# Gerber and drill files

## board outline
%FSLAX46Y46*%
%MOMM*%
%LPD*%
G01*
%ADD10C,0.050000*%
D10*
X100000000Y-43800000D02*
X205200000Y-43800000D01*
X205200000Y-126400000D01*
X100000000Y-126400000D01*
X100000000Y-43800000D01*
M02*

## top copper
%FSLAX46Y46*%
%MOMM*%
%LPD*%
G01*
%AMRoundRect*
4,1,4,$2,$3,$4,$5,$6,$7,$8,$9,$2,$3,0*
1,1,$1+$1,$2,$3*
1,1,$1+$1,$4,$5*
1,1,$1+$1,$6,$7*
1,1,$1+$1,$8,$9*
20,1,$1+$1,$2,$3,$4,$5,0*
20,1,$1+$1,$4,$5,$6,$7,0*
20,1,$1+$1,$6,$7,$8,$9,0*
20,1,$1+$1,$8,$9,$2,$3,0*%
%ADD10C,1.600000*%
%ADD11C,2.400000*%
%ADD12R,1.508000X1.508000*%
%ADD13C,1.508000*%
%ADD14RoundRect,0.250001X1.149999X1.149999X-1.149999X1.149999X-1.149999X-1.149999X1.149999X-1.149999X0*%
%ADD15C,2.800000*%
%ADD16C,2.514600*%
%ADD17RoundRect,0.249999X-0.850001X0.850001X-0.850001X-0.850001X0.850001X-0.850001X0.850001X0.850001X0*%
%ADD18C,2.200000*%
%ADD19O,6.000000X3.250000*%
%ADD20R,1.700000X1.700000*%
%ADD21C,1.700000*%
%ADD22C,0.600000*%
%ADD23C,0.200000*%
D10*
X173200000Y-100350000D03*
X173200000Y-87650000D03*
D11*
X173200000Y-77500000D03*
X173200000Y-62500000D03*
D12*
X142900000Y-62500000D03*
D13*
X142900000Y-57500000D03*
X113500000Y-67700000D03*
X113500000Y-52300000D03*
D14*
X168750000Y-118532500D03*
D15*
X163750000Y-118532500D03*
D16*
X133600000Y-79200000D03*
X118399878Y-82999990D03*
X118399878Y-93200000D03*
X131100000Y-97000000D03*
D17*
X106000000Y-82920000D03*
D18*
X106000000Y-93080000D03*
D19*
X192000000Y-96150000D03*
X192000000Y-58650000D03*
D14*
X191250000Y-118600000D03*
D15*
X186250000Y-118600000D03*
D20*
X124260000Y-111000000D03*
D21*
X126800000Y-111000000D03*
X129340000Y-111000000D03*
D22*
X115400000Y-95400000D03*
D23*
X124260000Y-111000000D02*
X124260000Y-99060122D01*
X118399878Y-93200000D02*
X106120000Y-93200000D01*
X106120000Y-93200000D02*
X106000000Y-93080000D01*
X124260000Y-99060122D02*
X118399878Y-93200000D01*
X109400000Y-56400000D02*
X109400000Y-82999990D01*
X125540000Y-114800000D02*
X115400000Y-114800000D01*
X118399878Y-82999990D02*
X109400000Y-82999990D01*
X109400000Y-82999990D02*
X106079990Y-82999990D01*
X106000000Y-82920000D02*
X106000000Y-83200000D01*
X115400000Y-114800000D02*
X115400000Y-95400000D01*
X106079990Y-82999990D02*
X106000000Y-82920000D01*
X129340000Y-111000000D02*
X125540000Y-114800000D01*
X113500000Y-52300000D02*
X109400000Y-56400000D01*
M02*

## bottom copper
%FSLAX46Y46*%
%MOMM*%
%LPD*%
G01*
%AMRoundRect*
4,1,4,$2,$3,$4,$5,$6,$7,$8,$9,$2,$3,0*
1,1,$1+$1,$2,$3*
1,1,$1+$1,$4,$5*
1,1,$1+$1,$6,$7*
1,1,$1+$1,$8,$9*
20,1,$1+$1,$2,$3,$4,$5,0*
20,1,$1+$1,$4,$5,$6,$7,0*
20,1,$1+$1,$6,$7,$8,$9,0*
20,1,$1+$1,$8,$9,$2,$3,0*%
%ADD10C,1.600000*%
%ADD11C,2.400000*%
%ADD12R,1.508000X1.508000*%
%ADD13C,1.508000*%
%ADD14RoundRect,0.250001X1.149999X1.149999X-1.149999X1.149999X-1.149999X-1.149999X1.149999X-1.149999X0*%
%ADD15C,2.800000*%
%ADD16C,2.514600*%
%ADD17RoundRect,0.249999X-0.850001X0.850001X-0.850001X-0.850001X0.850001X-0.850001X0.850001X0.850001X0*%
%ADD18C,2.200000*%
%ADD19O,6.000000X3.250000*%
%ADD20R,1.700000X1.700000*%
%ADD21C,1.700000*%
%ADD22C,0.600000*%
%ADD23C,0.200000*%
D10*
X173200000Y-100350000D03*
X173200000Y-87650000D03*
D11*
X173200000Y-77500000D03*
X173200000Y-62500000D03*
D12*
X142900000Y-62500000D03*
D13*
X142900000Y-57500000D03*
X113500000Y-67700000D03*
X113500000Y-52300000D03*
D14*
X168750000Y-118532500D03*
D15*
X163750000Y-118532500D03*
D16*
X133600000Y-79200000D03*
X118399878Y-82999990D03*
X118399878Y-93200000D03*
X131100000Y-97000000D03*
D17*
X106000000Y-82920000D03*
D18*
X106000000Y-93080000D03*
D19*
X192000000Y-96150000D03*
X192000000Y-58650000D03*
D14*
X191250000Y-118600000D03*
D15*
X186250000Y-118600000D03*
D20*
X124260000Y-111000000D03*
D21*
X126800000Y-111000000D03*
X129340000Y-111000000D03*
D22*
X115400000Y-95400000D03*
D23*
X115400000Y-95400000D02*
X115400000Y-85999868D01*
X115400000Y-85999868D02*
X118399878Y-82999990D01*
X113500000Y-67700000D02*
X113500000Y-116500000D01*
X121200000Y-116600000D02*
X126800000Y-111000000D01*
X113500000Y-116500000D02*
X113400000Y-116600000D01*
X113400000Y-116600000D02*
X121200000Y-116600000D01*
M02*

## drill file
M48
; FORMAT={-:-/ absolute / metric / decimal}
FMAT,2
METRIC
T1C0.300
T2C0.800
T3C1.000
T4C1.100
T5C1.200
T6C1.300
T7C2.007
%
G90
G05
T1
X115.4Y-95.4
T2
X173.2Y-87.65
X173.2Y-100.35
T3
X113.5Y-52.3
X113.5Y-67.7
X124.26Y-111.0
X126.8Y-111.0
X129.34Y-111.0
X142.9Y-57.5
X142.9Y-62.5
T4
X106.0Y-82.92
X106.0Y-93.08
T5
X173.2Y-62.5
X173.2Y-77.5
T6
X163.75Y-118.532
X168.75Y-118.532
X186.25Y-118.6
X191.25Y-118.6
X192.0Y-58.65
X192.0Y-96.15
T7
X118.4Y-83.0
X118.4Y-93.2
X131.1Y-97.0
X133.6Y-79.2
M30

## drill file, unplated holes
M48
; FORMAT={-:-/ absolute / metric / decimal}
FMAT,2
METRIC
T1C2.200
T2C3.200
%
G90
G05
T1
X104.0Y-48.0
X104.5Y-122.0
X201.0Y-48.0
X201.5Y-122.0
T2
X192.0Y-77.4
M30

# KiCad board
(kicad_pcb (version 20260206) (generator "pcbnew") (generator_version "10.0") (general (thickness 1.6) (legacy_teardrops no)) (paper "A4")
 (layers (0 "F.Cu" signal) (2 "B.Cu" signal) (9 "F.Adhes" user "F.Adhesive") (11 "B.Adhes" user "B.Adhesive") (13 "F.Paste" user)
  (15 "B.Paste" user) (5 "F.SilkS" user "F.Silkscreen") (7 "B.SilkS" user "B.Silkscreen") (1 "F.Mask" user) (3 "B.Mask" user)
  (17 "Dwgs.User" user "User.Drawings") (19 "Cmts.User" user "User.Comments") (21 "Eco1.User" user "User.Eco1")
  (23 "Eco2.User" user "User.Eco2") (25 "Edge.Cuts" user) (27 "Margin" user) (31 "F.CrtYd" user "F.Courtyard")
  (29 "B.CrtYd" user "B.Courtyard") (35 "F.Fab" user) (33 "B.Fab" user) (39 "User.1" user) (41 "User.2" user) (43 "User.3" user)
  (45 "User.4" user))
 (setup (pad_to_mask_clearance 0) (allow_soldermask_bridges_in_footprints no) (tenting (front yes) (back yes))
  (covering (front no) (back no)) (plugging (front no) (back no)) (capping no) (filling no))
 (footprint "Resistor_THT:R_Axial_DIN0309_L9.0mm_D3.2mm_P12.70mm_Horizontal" (layer "F.Cu") (at 173.2 100.35 90)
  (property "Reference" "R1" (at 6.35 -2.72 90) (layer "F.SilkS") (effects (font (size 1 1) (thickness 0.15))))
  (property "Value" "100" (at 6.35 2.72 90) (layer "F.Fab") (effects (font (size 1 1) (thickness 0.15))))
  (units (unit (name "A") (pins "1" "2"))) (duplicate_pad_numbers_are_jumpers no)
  (pad "1" thru_hole circle (at 0 0 90) (size 1.6 1.6) (drill 0.8) (layers "*.Cu" "*.Mask") (remove_unused_layers no) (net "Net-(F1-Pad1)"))
  (pad "2" thru_hole circle (at 12.7 0 90) (size 1.6 1.6) (drill 0.8) (layers "*.Cu" "*.Mask") (remove_unused_layers no)
   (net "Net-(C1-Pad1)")))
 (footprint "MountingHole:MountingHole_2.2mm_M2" (layer "F.Cu") (at 104.5 122)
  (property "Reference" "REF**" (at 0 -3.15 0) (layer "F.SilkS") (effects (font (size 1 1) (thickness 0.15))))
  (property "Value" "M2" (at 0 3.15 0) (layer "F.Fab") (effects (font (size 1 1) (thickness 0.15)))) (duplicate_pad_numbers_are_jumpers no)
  (pad "" np_thru_hole circle (at 0 0) (size 2.2 2.2) (drill 2.2) (layers "*.Cu" "*.Mask")))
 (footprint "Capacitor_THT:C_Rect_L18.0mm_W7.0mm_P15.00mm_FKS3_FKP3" (layer "F.Cu") (at 173.2 77.5 90)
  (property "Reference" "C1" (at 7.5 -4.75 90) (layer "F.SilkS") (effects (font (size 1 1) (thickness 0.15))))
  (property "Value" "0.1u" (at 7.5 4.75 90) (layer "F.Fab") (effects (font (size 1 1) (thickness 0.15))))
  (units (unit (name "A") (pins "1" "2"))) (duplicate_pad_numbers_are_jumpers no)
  (pad "1" thru_hole circle (at 0 0 90) (size 2.4 2.4) (drill 1.2) (layers "*.Cu" "*.Mask") (remove_unused_layers no) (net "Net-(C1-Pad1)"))
  (pad "2" thru_hole circle (at 15 0 90) (size 2.4 2.4) (drill 1.2) (layers "*.Cu" "*.Mask") (remove_unused_layers no)
   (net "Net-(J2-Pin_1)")))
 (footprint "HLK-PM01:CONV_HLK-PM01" (layer "F.Cu") (at 128.2 60 180)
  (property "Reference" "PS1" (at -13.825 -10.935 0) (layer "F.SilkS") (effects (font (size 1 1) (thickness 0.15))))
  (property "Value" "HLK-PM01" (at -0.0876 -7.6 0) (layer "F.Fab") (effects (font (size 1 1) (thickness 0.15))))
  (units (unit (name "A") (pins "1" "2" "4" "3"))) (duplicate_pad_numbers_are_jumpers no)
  (pad "1" thru_hole rect (at -14.7 -2.5 180) (size 1.508 1.508) (drill 1) (layers "*.Cu" "*.Mask") (remove_unused_layers no)
   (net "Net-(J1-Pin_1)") (solder_mask_margin 0.102))
  (pad "2" thru_hole circle (at -14.7 2.5 180) (size 1.508 1.508) (drill 1) (layers "*.Cu" "*.Mask") (remove_unused_layers no)
   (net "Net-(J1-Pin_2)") (solder_mask_margin 0.102))
  (pad "3" thru_hole circle (at 14.7 -7.7 180) (size 1.508 1.508) (drill 1) (layers "*.Cu" "*.Mask") (remove_unused_layers no)
   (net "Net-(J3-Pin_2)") (solder_mask_margin 0.102))
  (pad "4" thru_hole circle (at 14.7 7.7 180) (size 1.508 1.508) (drill 1) (layers "*.Cu" "*.Mask") (remove_unused_layers no)
   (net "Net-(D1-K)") (solder_mask_margin 0.102)))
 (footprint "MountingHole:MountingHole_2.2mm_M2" (layer "F.Cu") (at 104 48)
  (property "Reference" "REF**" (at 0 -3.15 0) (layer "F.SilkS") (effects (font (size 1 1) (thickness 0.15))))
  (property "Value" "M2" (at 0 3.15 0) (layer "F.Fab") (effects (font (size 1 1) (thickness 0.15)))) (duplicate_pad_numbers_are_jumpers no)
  (pad "" np_thru_hole circle (at 0 0) (size 2.2 2.2) (drill 2.2) (layers "*.Cu" "*.Mask")))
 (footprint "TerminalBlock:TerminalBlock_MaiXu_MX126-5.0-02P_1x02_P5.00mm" (layer "F.Cu") (at 168.75 118.5325 180)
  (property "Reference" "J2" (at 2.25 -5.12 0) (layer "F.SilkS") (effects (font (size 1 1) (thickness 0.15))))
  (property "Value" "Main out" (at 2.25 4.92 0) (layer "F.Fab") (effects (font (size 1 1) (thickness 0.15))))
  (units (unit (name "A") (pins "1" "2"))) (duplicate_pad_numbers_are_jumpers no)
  (pad "1" thru_hole roundrect (at 0 0 180) (size 2.8 2.8) (drill 1.3) (layers "*.Cu" "*.Mask") (remove_unused_layers no)
   (roundrect_rratio 0.089286) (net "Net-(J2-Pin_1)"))
  (pad "2" thru_hole circle (at 5 0 180) (size 2.8 2.8) (drill 1.3) (layers "*.Cu" "*.Mask") (remove_unused_layers no)
   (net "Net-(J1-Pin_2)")))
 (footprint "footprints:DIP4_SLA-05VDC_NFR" (layer "F.Cu") (at 133.6 79.2 -90)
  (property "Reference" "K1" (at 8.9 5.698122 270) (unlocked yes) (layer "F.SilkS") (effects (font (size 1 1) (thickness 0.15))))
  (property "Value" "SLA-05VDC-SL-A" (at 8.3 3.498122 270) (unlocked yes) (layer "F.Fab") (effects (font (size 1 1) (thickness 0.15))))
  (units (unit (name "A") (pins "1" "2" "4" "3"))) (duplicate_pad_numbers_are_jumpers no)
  (pad "1" thru_hole circle (at 0 0 270) (size 2.5146 2.5146) (drill 2.0066) (layers "*.Cu" "*.Mask") (remove_unused_layers no)
   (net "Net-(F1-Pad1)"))
  (pad "2" thru_hole circle (at 3.79999 15.200122 270) (size 2.5146 2.5146) (drill 2.0066) (layers "*.Cu" "*.Mask")
   (remove_unused_layers no) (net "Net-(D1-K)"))
  (pad "3" thru_hole circle (at 14 15.200122 270) (size 2.5146 2.5146) (drill 2.0066) (layers "*.Cu" "*.Mask") (remove_unused_layers no)
   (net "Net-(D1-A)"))
  (pad "4" thru_hole circle (at 17.8 2.5 270) (size 2.5146 2.5146) (drill 2.0066) (layers "*.Cu" "*.Mask") (remove_unused_layers no)
   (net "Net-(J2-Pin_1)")))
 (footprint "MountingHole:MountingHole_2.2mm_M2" (layer "F.Cu") (at 201.5 122)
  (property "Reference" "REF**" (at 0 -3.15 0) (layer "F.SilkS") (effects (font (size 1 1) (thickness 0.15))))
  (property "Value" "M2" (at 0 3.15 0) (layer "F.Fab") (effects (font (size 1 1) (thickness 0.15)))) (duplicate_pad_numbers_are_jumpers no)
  (pad "" np_thru_hole circle (at 0 0) (size 2.2 2.2) (drill 2.2) (layers "*.Cu" "*.Mask")))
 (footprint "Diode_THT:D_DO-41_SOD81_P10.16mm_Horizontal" (layer "F.Cu") (at 106 82.92 -90)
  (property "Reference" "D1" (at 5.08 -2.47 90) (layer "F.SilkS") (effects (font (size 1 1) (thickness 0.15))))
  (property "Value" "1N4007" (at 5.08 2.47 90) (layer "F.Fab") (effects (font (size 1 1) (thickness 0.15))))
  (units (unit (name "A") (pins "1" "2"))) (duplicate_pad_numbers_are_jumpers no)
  (pad "1" thru_hole roundrect (at 0 0 270) (size 2.2 2.2) (drill 1.1) (layers "*.Cu" "*.Mask") (remove_unused_layers no)
   (roundrect_rratio 0.113636) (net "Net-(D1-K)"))
  (pad "2" thru_hole circle (at 10.16 0 270) (size 2.2 2.2) (drill 1.1) (layers "*.Cu" "*.Mask") (remove_unused_layers no)
   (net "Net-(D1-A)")))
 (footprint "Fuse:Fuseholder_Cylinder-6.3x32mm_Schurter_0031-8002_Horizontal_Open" (layer "F.Cu") (at 192 96.15 90)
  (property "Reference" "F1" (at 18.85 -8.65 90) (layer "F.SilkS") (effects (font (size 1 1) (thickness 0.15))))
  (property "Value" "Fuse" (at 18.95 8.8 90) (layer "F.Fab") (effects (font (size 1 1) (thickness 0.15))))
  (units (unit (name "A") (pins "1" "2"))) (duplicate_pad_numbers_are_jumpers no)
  (pad "" np_thru_hole circle (at 18.75 0 90) (size 3.2 3.2) (drill 3.2) (layers "*.Cu" "*.Mask"))
  (pad "1" thru_hole oval (at 0 0 90) (size 3.25 6) (drill 1.3) (layers "*.Cu" "*.Mask") (remove_unused_layers no) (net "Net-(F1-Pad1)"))
  (pad "2" thru_hole oval (at 37.5 0 90) (size 3.25 6) (drill 1.3) (layers "*.Cu" "*.Mask") (remove_unused_layers no) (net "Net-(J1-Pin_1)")))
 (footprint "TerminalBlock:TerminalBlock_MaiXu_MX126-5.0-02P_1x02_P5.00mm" (layer "F.Cu") (at 191.25 118.6 180)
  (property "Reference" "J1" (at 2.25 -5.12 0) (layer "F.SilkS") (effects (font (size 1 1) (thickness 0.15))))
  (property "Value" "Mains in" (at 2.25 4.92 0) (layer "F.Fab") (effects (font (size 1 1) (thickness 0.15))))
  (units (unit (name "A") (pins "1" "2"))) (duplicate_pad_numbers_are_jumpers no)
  (pad "1" thru_hole roundrect (at 0 0 180) (size 2.8 2.8) (drill 1.3) (layers "*.Cu" "*.Mask") (remove_unused_layers no)
   (roundrect_rratio 0.089286) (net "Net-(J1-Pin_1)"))
  (pad "2" thru_hole circle (at 5 0 180) (size 2.8 2.8) (drill 1.3) (layers "*.Cu" "*.Mask") (remove_unused_layers no)
   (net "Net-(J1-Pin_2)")))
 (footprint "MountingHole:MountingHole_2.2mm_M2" (layer "F.Cu") (at 201 48)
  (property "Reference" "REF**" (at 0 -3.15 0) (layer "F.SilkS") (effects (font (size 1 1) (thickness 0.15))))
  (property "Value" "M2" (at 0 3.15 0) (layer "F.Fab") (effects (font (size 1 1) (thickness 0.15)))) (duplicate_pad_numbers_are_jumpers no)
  (pad "" np_thru_hole circle (at 0 0) (size 2.2 2.2) (drill 2.2) (layers "*.Cu" "*.Mask")))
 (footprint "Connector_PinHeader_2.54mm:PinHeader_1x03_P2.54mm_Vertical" (layer "F.Cu") (at 124.26 111 90)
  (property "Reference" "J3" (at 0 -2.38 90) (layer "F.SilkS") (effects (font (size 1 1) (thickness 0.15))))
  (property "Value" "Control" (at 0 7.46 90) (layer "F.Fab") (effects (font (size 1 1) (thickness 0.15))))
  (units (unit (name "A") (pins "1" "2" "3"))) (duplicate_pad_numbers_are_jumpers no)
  (pad "1" thru_hole rect (at 0 0 90) (size 1.7 1.7) (drill 1) (layers "*.Cu" "*.Mask") (remove_unused_layers no) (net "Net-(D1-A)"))
  (pad "2" thru_hole circle (at 0 2.54 90) (size 1.7 1.7) (drill 1) (layers "*.Cu" "*.Mask") (remove_unused_layers no)
   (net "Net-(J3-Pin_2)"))
  (pad "3" thru_hole circle (at 0 5.08 90) (size 1.7 1.7) (drill 1) (layers "*.Cu" "*.Mask") (remove_unused_layers no) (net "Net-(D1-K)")))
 (gr_rect (start 100 43.8) (end 205.2 126.4) (stroke (width 0.05) (type default)) (fill no) (layer "Edge.Cuts"))
 (segment (start 113.5 67.7) (end 113.5 116.5) (width 0.2) (layer "B.Cu") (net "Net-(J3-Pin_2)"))
 (segment (start 121.2 116.6) (end 126.8 111) (width 0.2) (layer "B.Cu") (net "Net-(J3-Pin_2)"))
 (segment (start 113.5 116.5) (end 113.4 116.6) (width 0.2) (layer "B.Cu") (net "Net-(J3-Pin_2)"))
 (segment (start 113.4 116.6) (end 121.2 116.6) (width 0.2) (layer "B.Cu") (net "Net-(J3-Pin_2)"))
 (segment (start 109.4 56.4) (end 109.4 82.99999) (width 0.2) (layer "F.Cu") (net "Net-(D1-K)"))
 (segment (start 125.54 114.8) (end 115.4 114.8) (width 0.2) (layer "F.Cu") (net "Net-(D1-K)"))
 (segment (start 118.399878 82.99999) (end 109.4 82.99999) (width 0.2) (layer "F.Cu") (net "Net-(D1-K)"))
 (segment (start 109.4 82.99999) (end 106.07999 82.99999) (width 0.2) (layer "F.Cu") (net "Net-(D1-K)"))
 (segment (start 106 82.92) (end 106 83.2) (width 0.2) (layer "F.Cu") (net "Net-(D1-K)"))
 (segment (start 115.4 114.8) (end 115.4 95.4) (width 0.2) (layer "F.Cu") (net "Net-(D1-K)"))
 (segment (start 106.07999 82.99999) (end 106 82.92) (width 0.2) (layer "F.Cu") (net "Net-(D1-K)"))
 (segment (start 129.34 111) (end 125.54 114.8) (width 0.2) (layer "F.Cu") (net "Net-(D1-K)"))
 (segment (start 113.5 52.3) (end 109.4 56.4) (width 0.2) (layer "F.Cu") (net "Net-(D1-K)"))
 (via (at 115.4 95.4) (size 0.6) (drill 0.3) (layers "F.Cu" "B.Cu") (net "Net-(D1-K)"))
 (segment (start 115.4 95.4) (end 115.4 85.999868) (width 0.2) (layer "B.Cu") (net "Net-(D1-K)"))
 (segment (start 115.4 85.999868) (end 118.399878 82.99999) (width 0.2) (layer "B.Cu") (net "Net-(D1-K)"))
 (segment (start 124.26 111) (end 124.26 99.060122) (width 0.2) (layer "F.Cu") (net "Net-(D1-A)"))
 (segment (start 118.399878 93.2) (end 106.12 93.2) (width 0.2) (layer "F.Cu") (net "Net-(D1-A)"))
 (segment (start 106.12 93.2) (end 106 93.08) (width 0.2) (layer "F.Cu") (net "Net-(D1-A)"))
 (segment (start 124.26 99.060122) (end 118.399878 93.2) (width 0.2) (layer "F.Cu") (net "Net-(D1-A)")))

